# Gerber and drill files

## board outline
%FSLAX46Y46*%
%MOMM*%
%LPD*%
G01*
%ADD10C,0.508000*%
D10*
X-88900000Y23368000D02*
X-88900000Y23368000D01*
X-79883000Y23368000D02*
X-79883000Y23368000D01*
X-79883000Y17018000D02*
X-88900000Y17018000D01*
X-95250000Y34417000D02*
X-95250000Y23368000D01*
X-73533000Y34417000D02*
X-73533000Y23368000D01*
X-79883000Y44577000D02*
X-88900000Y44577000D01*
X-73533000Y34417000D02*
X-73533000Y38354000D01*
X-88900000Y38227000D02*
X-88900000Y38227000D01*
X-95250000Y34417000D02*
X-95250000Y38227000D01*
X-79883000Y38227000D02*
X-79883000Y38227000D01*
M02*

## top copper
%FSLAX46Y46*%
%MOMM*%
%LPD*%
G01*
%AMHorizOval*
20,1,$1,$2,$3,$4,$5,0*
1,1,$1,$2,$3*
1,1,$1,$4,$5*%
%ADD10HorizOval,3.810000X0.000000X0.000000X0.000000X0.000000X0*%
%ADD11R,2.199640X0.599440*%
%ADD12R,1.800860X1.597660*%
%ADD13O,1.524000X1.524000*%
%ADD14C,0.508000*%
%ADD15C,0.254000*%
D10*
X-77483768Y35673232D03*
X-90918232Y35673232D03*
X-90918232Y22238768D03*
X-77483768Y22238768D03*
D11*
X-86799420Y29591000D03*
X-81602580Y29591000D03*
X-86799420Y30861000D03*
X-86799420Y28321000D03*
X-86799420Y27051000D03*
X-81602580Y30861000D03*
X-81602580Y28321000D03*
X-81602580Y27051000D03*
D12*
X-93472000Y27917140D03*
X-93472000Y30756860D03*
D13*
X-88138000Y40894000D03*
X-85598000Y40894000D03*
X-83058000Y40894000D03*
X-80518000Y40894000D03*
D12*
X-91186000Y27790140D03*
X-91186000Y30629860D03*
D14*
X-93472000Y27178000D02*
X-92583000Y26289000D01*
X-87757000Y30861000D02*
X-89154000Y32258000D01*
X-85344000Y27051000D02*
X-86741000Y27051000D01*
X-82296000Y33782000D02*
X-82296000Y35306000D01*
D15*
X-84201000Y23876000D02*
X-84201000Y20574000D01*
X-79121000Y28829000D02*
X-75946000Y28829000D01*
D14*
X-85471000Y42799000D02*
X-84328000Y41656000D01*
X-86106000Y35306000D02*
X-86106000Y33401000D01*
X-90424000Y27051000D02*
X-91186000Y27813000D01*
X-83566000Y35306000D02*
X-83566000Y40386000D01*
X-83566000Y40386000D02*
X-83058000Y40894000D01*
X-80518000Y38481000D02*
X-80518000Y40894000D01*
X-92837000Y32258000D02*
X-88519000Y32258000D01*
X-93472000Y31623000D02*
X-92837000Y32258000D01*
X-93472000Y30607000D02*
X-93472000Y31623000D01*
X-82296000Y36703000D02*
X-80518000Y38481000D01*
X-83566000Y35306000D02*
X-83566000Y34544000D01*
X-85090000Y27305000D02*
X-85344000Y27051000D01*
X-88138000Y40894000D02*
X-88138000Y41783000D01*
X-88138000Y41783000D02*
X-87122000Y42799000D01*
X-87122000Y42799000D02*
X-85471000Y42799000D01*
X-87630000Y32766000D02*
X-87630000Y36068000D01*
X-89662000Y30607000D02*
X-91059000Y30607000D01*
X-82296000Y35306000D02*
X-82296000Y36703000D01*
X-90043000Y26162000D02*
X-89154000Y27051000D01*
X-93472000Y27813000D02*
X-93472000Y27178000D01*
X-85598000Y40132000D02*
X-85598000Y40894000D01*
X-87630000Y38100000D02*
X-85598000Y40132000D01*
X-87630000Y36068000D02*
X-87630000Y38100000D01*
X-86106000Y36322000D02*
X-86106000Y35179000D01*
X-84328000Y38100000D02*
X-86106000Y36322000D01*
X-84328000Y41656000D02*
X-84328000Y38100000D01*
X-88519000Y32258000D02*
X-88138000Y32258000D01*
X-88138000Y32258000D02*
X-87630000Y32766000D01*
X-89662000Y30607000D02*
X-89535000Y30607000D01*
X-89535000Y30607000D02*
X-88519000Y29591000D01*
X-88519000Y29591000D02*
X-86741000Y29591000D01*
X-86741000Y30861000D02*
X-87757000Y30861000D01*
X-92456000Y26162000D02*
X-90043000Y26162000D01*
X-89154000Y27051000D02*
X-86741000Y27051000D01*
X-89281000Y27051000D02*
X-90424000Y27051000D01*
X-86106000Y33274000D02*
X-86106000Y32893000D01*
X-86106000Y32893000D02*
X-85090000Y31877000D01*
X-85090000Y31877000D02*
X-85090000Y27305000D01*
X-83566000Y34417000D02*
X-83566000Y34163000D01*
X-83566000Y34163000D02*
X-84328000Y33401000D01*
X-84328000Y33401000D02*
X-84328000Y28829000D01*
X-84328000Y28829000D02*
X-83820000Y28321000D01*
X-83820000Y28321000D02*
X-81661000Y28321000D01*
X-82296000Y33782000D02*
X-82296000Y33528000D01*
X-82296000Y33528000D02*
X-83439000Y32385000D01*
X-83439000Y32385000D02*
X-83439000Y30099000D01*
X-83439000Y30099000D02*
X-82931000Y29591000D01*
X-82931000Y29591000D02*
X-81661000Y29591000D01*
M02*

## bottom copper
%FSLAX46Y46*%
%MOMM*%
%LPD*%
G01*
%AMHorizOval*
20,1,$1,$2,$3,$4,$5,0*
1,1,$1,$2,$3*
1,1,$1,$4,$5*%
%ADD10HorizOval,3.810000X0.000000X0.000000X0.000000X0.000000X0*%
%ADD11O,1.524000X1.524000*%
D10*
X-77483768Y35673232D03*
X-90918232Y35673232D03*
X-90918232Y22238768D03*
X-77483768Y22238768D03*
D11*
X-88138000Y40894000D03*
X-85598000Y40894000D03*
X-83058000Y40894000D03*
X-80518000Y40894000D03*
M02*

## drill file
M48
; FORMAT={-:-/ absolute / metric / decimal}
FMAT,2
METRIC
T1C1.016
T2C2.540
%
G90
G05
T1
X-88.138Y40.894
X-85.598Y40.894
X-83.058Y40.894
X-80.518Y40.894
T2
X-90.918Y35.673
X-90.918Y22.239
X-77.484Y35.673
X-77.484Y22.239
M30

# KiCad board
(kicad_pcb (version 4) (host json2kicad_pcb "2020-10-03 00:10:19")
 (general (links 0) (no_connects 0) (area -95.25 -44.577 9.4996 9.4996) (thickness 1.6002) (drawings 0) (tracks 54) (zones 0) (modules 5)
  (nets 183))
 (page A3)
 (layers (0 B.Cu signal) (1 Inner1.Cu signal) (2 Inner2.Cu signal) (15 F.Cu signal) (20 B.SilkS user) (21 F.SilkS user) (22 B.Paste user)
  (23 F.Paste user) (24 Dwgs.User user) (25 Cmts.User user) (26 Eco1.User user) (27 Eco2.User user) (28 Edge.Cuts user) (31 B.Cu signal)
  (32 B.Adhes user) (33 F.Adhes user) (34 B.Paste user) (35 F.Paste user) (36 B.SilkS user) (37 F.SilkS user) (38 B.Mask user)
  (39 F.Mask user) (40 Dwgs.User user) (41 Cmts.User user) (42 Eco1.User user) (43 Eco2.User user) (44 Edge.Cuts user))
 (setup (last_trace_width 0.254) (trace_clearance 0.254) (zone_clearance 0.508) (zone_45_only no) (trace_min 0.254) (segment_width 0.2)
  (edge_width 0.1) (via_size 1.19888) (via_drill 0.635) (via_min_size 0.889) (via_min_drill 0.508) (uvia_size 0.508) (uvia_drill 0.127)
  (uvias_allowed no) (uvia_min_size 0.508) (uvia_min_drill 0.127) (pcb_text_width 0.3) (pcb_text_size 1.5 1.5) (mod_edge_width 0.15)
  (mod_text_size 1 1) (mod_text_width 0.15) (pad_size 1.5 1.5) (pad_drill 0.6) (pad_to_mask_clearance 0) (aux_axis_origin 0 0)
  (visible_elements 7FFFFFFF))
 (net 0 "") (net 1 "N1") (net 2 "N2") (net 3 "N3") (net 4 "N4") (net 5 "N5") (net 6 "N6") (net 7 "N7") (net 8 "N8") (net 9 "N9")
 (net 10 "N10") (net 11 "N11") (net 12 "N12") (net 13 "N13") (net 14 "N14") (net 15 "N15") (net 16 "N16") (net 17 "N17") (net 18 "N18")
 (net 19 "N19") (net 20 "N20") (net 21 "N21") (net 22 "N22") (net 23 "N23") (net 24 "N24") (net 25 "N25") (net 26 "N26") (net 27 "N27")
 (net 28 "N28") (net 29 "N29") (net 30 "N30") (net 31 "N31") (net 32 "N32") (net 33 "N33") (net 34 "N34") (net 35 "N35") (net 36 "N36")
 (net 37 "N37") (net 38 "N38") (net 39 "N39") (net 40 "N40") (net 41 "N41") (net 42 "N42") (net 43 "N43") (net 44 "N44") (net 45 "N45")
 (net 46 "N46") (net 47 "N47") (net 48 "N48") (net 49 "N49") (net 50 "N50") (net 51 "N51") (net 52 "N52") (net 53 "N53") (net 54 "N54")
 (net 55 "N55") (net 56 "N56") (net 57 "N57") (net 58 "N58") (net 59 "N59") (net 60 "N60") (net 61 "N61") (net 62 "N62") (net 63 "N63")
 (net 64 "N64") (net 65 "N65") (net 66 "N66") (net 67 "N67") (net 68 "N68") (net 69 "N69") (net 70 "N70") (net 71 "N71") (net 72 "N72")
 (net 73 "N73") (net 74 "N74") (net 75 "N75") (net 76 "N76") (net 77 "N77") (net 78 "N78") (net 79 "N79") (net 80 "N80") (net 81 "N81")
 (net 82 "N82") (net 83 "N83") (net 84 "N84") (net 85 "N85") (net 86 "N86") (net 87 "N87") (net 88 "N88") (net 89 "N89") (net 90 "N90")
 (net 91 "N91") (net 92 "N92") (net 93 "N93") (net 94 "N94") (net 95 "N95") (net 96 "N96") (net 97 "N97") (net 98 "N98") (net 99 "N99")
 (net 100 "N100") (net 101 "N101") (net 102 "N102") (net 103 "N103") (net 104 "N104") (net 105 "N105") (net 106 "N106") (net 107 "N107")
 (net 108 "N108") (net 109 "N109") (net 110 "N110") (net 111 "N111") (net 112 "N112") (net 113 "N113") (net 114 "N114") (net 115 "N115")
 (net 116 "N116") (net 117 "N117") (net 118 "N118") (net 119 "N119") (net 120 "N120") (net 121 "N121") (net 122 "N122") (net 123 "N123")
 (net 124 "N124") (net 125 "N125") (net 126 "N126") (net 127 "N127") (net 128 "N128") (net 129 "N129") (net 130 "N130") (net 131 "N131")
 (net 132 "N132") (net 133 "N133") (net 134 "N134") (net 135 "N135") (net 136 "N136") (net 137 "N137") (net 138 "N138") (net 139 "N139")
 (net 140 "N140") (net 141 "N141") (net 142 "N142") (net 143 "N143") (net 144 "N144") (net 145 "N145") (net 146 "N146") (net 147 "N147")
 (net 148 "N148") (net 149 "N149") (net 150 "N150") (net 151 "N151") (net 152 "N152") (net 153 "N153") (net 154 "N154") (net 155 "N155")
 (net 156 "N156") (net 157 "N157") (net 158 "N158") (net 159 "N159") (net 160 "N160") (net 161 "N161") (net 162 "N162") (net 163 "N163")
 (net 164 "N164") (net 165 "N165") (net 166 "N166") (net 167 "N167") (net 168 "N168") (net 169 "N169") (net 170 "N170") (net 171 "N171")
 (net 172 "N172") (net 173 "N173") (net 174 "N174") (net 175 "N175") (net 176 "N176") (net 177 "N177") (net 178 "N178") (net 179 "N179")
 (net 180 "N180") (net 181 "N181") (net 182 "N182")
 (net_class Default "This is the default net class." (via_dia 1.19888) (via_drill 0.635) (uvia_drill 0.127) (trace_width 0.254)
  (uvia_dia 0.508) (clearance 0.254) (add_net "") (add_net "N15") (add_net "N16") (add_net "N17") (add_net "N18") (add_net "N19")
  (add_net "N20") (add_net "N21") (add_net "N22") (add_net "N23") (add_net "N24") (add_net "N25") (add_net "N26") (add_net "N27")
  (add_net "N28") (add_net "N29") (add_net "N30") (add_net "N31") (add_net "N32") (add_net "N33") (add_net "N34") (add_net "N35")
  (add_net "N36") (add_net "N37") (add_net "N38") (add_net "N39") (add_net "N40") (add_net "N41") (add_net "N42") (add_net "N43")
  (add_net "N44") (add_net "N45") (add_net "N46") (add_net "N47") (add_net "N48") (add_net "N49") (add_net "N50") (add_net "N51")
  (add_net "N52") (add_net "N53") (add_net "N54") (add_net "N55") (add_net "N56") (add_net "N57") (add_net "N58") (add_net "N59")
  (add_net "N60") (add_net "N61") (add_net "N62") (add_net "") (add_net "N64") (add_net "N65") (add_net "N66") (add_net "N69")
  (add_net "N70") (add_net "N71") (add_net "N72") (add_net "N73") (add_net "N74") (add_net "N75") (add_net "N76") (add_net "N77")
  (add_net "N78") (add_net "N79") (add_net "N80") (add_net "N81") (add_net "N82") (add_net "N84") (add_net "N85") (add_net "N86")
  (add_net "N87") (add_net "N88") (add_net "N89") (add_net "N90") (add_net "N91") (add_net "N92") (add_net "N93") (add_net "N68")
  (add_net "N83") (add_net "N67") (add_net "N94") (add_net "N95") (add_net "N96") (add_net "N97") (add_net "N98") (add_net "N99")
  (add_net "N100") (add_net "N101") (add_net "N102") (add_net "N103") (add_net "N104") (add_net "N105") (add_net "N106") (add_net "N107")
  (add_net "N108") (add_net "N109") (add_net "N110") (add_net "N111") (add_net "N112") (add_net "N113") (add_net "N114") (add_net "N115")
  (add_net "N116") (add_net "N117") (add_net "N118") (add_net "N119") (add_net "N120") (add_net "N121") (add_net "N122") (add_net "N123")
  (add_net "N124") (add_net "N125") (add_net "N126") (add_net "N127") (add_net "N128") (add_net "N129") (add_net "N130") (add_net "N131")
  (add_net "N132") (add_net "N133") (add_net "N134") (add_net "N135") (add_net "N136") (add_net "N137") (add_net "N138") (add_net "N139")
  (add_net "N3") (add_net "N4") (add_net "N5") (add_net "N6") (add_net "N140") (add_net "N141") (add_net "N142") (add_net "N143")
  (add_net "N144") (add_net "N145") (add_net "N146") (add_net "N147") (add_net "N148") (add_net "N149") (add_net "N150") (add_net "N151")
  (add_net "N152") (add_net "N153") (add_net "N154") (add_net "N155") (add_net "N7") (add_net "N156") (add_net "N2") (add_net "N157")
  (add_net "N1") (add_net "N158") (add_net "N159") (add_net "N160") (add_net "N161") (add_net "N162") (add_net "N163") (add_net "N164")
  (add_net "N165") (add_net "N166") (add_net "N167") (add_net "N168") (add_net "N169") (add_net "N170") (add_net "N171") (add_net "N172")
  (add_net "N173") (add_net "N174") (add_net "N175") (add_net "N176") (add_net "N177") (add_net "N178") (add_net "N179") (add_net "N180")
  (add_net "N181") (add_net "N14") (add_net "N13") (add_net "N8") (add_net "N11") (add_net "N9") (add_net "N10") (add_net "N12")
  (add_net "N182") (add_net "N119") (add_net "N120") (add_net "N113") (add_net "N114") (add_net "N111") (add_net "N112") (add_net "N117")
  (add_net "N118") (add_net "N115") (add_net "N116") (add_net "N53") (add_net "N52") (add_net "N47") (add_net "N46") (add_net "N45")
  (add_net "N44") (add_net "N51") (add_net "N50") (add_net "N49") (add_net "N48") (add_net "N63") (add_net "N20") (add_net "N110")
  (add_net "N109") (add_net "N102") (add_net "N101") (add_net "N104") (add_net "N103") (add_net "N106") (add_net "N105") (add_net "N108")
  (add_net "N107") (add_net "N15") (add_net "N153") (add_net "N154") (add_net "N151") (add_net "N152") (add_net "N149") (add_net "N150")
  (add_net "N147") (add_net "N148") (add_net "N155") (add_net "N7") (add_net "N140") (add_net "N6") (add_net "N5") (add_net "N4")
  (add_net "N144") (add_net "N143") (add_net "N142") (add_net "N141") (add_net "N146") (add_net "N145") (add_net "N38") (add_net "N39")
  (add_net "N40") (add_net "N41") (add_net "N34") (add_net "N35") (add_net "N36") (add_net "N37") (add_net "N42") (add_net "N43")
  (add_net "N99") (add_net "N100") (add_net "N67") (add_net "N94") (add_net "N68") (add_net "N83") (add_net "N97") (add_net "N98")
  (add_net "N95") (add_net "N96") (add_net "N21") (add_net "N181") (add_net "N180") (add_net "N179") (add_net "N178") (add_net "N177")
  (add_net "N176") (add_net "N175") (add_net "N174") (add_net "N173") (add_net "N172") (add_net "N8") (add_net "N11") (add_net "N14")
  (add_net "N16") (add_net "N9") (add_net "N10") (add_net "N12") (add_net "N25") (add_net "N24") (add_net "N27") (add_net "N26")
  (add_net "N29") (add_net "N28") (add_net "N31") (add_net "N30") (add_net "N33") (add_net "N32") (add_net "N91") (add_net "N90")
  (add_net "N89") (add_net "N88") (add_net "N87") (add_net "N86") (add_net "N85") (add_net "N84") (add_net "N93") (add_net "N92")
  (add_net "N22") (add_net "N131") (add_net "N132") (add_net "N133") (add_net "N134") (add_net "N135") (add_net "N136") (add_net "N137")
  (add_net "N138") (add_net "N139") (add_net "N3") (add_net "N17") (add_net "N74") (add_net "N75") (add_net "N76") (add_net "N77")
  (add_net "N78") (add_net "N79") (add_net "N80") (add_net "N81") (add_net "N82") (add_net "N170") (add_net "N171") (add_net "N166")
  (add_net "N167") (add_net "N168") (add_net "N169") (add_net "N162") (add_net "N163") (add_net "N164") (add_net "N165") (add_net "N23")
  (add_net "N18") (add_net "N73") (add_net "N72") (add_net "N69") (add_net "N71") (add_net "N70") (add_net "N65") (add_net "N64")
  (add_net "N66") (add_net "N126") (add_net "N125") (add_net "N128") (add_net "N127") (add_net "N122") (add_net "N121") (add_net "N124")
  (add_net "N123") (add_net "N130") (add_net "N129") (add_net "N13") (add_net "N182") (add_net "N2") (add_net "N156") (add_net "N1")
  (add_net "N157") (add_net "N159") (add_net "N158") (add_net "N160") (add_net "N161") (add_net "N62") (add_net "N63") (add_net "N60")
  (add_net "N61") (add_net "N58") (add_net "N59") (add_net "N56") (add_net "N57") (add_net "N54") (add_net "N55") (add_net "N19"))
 (segment (start -93.472 -27.178) (end -92.583 -26.289) (width 0.508) (layer F.Cu) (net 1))
 (gr_line (start -88.9 -23.368) (end -88.9 -23.368) (angle -90.00) (width 0.508) (layer Edge.Cuts))
 (gr_line (start -79.883 -23.368) (end -79.883 -23.368) (angle -90.00) (width 0.508) (layer Edge.Cuts))
 (segment (start -87.757 -30.861) (end -89.154 -32.258) (width 0.508) (layer F.Cu) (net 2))
 (gr_line (start -79.883 -17.018) (end -88.9 -17.018) (angle 51566.20) (width 0.508) (layer Edge.Cuts))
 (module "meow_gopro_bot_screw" (layer "F.Cu") (at -84.201 -28.956 135.00)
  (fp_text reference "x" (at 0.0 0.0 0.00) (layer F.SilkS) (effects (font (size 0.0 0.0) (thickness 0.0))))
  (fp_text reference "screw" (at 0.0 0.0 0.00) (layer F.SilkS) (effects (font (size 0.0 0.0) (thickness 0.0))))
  (pad S0 thru_hole oval (at 0.0 9.4996 135.00) (size 3.81 3.81) (drill 2.54)
   (layers "B.Cu" "Inner1.Cu" "Inner2.Cu" "F.Cu" "B.Paste" "F.Paste") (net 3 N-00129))
  (pad S1 thru_hole oval (at 9.4996 0.0 135.00) (size 3.81 3.81) (drill 2.54)
   (layers "B.Cu" "Inner1.Cu" "Inner2.Cu" "F.Cu" "B.Paste" "F.Paste") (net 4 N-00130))
  (pad S2 thru_hole oval (at 0.0 -9.4996 135.00) (size 3.81 3.81) (drill 2.54)
   (layers "B.Cu" "Inner1.Cu" "Inner2.Cu" "F.Cu" "B.Paste" "F.Paste") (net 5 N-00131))
  (pad S3 thru_hole oval (at -9.4996 0.0 135.00) (size 3.81 3.81) (drill 2.54)
   (layers "B.Cu" "Inner1.Cu" "Inner2.Cu" "F.Cu" "B.Paste" "F.Paste") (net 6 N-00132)))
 (gr_line (start -95.25 -34.417) (end -95.25 -23.368) (angle 51566.20) (width 0.508) (layer Edge.Cuts))
 (gr_line (start -73.533 -34.417) (end -73.533 -23.368) (angle 51566.20) (width 0.508) (layer Edge.Cuts))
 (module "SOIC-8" (layer "F.Cu") (at -84.201 -28.956 -90.00)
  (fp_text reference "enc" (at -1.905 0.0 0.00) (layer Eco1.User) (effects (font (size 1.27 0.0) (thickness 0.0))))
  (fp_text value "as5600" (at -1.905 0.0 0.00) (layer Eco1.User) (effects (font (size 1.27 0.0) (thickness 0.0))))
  (pad 2 smd rect (at -0.635 2.59842 -90.00) (size 0.59944 2.19964) (drill 0.0) (layers "F.Cu" "F.Paste") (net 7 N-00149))
  (pad 7 smd rect (at -0.635 -2.59842 -90.00) (size 0.59944 2.19964) (drill 0.0) (layers "F.Cu" "F.Paste") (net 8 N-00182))
  (pad 1 smd rect (at -1.905 2.59842 -90.00) (size 0.59944 2.19964) (drill 0.0) (layers "F.Cu" "F.Paste") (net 2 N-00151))
  (pad 3 smd rect (at 0.635 2.59842 -90.00) (size 0.59944 2.19964) (drill 0.0) (layers "F.Cu" "F.Paste") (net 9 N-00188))
  (pad 4 smd rect (at 1.905 2.59842 -90.00) (size 0.59944 2.19964) (drill 0.0) (layers "F.Cu" "F.Paste") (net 1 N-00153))
  (pad 8 smd rect (at -1.905 -2.59842 -90.00) (size 0.59944 2.19964) (drill 0.0) (layers "F.Cu" "F.Paste") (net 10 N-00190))
  (pad 6 smd rect (at 0.635 -2.59842 -90.00) (size 0.59944 2.19964) (drill 0.0) (layers "F.Cu" "F.Paste") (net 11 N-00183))
  (pad 5 smd rect (at 1.905 -2.59842 -90.00) (size 0.59944 2.19964) (drill 0.0) (layers "F.Cu" "F.Paste") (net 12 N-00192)))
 (gr_line (start -79.883 -44.577) (end -88.9 -44.577) (angle 51566.20) (width 0.508) (layer Edge.Cuts))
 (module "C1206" (layer "F.Cu") (at -93.472 -29.337 -90.00)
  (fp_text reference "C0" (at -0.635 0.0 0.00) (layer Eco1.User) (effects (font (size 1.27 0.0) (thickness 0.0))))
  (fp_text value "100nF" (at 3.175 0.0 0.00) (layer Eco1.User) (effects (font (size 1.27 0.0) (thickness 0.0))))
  (pad 2 smd rect (at 1.41986 0.0 -90.00) (size 1.59766 1.80086) (drill 0.0) (layers "F.Cu" "F.Paste") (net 1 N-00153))
  (pad 1 smd rect (at -1.41986 0.0 -90.00) (size 1.59766 1.80086) (drill 0.0) (layers "F.Cu" "F.Paste") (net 2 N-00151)))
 (segment (start -85.344 -27.051) (end -86.741 -27.051) (width 0.508) (layer F.Cu) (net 1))
 (segment (start -82.296 -33.782) (end -82.296 -35.306) (width 0.508) (layer F.Cu) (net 8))
 (segment (start -84.201 -23.876) (end -84.201 -20.574) (width 0.254) (layer F.Cu) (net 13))
 (segment (start -79.121 -28.829) (end -75.946 -28.829) (width 0.254) (layer F.Cu) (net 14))
 (segment (start -85.471 -42.799) (end -84.328 -41.656) (width 0.508) (layer F.Cu) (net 1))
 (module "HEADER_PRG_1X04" (layer "F.Cu") (at -84.328 -40.894 0.00)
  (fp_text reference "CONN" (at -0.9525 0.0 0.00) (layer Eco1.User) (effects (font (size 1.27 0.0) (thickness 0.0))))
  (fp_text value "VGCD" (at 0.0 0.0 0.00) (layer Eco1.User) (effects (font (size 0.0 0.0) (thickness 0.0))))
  (pad 1 thru_hole oval (at -3.81 0.0 0.00) (size 1.524 1.524) (drill 1.016)
   (layers "B.Cu" "Inner1.Cu" "Inner2.Cu" "F.Cu" "B.Paste" "F.Paste") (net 1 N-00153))
  (pad 2 thru_hole oval (at -1.27 0.0 0.00) (size 1.524 1.524) (drill 1.016)
   (layers "B.Cu" "Inner1.Cu" "Inner2.Cu" "F.Cu" "B.Paste" "F.Paste") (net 2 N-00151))
  (pad 3 thru_hole oval (at 1.27 0.0 0.00) (size 1.524 1.524) (drill 1.016)
   (layers "B.Cu" "Inner1.Cu" "Inner2.Cu" "F.Cu" "B.Paste" "F.Paste") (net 11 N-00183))
  (pad 4 thru_hole oval (at 3.81 0.0 0.00) (size 1.524 1.524) (drill 1.016)
   (layers "B.Cu" "Inner1.Cu" "Inner2.Cu" "F.Cu" "B.Paste" "F.Paste") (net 8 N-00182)))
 (segment (start -86.106 -35.306) (end -86.106 -33.401) (width 0.508) (layer F.Cu) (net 1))
 (segment (start -90.424 -27.051) (end -91.186 -27.813) (width 0.508) (layer F.Cu) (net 1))
 (segment (start -83.566 -35.306) (end -83.566 -40.386) (width 0.508) (layer F.Cu) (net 11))
 (segment (start -83.566 -40.386) (end -83.058 -40.894) (width 0.508) (layer F.Cu) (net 11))
 (segment (start -80.518 -38.481) (end -80.518 -40.894) (width 0.508) (layer F.Cu) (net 8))
 (segment (start -92.837 -32.258) (end -88.519 -32.258) (width 0.508) (layer F.Cu) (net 2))
 (segment (start -93.472 -31.623) (end -92.837 -32.258) (width 0.508) (layer F.Cu) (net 2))
 (segment (start -93.472 -30.607) (end -93.472 -31.623) (width 0.508) (layer F.Cu) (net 2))
 (segment (start -82.296 -36.703) (end -80.518 -38.481) (width 0.508) (layer F.Cu) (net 8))
 (gr_line (start -73.533 -34.417) (end -73.533 -38.354) (angle 51566.20) (width 0.508) (layer Edge.Cuts))
 (gr_line (start -88.9 -38.227) (end -88.9 -38.227) (angle -90.00) (width 0.508) (layer Edge.Cuts))
 (segment (start -83.566 -35.306) (end -83.566 -34.544) (width 0.508) (layer F.Cu) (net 11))
 (segment (start -85.09 -27.305) (end -85.344 -27.051) (width 0.508) (layer F.Cu) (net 1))
 (segment (start -88.138 -40.894) (end -88.138 -41.783) (width 0.508) (layer F.Cu) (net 1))
 (segment (start -88.138 -41.783) (end -87.122 -42.799) (width 0.508) (layer F.Cu) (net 1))
 (segment (start -87.122 -42.799) (end -85.471 -42.799) (width 0.508) (layer F.Cu) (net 1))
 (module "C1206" (layer "F.Cu") (at -91.186 -29.21 -90.00)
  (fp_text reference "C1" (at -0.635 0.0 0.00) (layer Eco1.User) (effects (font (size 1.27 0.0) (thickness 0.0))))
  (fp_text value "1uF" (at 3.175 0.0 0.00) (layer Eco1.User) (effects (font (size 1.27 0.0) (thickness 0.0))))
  (pad 2 smd rect (at 1.41986 0.0 -90.00) (size 1.59766 1.80086) (drill 0.0) (layers "F.Cu" "F.Paste") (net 1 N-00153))
  (pad 1 smd rect (at -1.41986 0.0 -90.00) (size 1.59766 1.80086) (drill 0.0) (layers "F.Cu" "F.Paste") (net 7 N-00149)))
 (gr_line (start -95.25 -34.417) (end -95.25 -38.227) (angle 51566.20) (width 0.508) (layer Edge.Cuts))
 (segment (start -87.63 -32.766) (end -87.63 -36.068) (width 0.508) (layer F.Cu) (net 2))
 (segment (start -89.662 -30.607) (end -91.059 -30.607) (width 0.508) (layer F.Cu) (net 7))
 (segment (start -82.296 -35.306) (end -82.296 -36.703) (width 0.508) (layer F.Cu) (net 8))
 (segment (start -90.043 -26.162) (end -89.154 -27.051) (width 0.508) (layer F.Cu) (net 1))
 (segment (start -93.472 -27.813) (end -93.472 -27.178) (width 0.508) (layer F.Cu) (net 1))
 (segment (start -85.598 -40.132) (end -85.598 -40.894) (width 0.508) (layer F.Cu) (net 2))
 (segment (start -87.63 -38.1) (end -85.598 -40.132) (width 0.508) (layer F.Cu) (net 2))
 (segment (start -87.63 -36.068) (end -87.63 -38.1) (width 0.508) (layer F.Cu) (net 2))
 (segment (start -86.106 -36.322) (end -86.106 -35.179) (width 0.508) (layer F.Cu) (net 1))
 (gr_line (start -79.883 -38.227) (end -79.883 -38.227) (angle -90.00) (width 0.508) (layer Edge.Cuts))
 (segment (start -84.328 -38.1) (end -86.106 -36.322) (width 0.508) (layer F.Cu) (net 1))
 (segment (start -84.328 -41.656) (end -84.328 -38.1) (width 0.508) (layer F.Cu) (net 1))
 (segment (start -88.519 -32.258) (end -88.138 -32.258) (width 0.508) (layer F.Cu) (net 2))
 (segment (start -88.138 -32.258) (end -87.63 -32.766) (width 0.508) (layer F.Cu) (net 2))
 (segment (start -89.662 -30.607) (end -89.535 -30.607) (width 0.508) (layer F.Cu) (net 7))
 (segment (start -89.535 -30.607) (end -88.519 -29.591) (width 0.508) (layer F.Cu) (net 7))
 (segment (start -88.519 -29.591) (end -86.741 -29.591) (width 0.508) (layer F.Cu) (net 7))
 (segment (start -86.741 -30.861) (end -87.757 -30.861) (width 0.508) (layer F.Cu) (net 2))
 (segment (start -92.456 -26.162) (end -90.043 -26.162) (width 0.508) (layer F.Cu) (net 1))
 (segment (start -89.154 -27.051) (end -86.741 -27.051) (width 0.508) (layer F.Cu) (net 1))
 (segment (start -89.281 -27.051) (end -90.424 -27.051) (width 0.508) (layer F.Cu) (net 1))
 (segment (start -86.106 -33.274) (end -86.106 -32.893) (width 0.508) (layer F.Cu) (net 1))
 (segment (start -86.106 -32.893) (end -85.09 -31.877) (width 0.508) (layer F.Cu) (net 1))
 (segment (start -85.09 -31.877) (end -85.09 -27.305) (width 0.508) (layer F.Cu) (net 1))
 (segment (start -83.566 -34.417) (end -83.566 -34.163) (width 0.508) (layer F.Cu) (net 11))
 (segment (start -83.566 -34.163) (end -84.328 -33.401) (width 0.508) (layer F.Cu) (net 11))
 (segment (start -84.328 -33.401) (end -84.328 -28.829) (width 0.508) (layer F.Cu) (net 11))
 (segment (start -84.328 -28.829) (end -83.82 -28.321) (width 0.508) (layer F.Cu) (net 11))
 (segment (start -83.82 -28.321) (end -81.661 -28.321) (width 0.508) (layer F.Cu) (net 11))
 (segment (start -82.296 -33.782) (end -82.296 -33.528) (width 0.508) (layer F.Cu) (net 8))
 (segment (start -82.296 -33.528) (end -83.439 -32.385) (width 0.508) (layer F.Cu) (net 8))
 (segment (start -83.439 -32.385) (end -83.439 -30.099) (width 0.508) (layer F.Cu) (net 8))
 (segment (start -83.439 -30.099) (end -82.931 -29.591) (width 0.508) (layer F.Cu) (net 8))
 (segment (start -82.931 -29.591) (end -81.661 -29.591) (width 0.508) (layer F.Cu) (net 8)))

